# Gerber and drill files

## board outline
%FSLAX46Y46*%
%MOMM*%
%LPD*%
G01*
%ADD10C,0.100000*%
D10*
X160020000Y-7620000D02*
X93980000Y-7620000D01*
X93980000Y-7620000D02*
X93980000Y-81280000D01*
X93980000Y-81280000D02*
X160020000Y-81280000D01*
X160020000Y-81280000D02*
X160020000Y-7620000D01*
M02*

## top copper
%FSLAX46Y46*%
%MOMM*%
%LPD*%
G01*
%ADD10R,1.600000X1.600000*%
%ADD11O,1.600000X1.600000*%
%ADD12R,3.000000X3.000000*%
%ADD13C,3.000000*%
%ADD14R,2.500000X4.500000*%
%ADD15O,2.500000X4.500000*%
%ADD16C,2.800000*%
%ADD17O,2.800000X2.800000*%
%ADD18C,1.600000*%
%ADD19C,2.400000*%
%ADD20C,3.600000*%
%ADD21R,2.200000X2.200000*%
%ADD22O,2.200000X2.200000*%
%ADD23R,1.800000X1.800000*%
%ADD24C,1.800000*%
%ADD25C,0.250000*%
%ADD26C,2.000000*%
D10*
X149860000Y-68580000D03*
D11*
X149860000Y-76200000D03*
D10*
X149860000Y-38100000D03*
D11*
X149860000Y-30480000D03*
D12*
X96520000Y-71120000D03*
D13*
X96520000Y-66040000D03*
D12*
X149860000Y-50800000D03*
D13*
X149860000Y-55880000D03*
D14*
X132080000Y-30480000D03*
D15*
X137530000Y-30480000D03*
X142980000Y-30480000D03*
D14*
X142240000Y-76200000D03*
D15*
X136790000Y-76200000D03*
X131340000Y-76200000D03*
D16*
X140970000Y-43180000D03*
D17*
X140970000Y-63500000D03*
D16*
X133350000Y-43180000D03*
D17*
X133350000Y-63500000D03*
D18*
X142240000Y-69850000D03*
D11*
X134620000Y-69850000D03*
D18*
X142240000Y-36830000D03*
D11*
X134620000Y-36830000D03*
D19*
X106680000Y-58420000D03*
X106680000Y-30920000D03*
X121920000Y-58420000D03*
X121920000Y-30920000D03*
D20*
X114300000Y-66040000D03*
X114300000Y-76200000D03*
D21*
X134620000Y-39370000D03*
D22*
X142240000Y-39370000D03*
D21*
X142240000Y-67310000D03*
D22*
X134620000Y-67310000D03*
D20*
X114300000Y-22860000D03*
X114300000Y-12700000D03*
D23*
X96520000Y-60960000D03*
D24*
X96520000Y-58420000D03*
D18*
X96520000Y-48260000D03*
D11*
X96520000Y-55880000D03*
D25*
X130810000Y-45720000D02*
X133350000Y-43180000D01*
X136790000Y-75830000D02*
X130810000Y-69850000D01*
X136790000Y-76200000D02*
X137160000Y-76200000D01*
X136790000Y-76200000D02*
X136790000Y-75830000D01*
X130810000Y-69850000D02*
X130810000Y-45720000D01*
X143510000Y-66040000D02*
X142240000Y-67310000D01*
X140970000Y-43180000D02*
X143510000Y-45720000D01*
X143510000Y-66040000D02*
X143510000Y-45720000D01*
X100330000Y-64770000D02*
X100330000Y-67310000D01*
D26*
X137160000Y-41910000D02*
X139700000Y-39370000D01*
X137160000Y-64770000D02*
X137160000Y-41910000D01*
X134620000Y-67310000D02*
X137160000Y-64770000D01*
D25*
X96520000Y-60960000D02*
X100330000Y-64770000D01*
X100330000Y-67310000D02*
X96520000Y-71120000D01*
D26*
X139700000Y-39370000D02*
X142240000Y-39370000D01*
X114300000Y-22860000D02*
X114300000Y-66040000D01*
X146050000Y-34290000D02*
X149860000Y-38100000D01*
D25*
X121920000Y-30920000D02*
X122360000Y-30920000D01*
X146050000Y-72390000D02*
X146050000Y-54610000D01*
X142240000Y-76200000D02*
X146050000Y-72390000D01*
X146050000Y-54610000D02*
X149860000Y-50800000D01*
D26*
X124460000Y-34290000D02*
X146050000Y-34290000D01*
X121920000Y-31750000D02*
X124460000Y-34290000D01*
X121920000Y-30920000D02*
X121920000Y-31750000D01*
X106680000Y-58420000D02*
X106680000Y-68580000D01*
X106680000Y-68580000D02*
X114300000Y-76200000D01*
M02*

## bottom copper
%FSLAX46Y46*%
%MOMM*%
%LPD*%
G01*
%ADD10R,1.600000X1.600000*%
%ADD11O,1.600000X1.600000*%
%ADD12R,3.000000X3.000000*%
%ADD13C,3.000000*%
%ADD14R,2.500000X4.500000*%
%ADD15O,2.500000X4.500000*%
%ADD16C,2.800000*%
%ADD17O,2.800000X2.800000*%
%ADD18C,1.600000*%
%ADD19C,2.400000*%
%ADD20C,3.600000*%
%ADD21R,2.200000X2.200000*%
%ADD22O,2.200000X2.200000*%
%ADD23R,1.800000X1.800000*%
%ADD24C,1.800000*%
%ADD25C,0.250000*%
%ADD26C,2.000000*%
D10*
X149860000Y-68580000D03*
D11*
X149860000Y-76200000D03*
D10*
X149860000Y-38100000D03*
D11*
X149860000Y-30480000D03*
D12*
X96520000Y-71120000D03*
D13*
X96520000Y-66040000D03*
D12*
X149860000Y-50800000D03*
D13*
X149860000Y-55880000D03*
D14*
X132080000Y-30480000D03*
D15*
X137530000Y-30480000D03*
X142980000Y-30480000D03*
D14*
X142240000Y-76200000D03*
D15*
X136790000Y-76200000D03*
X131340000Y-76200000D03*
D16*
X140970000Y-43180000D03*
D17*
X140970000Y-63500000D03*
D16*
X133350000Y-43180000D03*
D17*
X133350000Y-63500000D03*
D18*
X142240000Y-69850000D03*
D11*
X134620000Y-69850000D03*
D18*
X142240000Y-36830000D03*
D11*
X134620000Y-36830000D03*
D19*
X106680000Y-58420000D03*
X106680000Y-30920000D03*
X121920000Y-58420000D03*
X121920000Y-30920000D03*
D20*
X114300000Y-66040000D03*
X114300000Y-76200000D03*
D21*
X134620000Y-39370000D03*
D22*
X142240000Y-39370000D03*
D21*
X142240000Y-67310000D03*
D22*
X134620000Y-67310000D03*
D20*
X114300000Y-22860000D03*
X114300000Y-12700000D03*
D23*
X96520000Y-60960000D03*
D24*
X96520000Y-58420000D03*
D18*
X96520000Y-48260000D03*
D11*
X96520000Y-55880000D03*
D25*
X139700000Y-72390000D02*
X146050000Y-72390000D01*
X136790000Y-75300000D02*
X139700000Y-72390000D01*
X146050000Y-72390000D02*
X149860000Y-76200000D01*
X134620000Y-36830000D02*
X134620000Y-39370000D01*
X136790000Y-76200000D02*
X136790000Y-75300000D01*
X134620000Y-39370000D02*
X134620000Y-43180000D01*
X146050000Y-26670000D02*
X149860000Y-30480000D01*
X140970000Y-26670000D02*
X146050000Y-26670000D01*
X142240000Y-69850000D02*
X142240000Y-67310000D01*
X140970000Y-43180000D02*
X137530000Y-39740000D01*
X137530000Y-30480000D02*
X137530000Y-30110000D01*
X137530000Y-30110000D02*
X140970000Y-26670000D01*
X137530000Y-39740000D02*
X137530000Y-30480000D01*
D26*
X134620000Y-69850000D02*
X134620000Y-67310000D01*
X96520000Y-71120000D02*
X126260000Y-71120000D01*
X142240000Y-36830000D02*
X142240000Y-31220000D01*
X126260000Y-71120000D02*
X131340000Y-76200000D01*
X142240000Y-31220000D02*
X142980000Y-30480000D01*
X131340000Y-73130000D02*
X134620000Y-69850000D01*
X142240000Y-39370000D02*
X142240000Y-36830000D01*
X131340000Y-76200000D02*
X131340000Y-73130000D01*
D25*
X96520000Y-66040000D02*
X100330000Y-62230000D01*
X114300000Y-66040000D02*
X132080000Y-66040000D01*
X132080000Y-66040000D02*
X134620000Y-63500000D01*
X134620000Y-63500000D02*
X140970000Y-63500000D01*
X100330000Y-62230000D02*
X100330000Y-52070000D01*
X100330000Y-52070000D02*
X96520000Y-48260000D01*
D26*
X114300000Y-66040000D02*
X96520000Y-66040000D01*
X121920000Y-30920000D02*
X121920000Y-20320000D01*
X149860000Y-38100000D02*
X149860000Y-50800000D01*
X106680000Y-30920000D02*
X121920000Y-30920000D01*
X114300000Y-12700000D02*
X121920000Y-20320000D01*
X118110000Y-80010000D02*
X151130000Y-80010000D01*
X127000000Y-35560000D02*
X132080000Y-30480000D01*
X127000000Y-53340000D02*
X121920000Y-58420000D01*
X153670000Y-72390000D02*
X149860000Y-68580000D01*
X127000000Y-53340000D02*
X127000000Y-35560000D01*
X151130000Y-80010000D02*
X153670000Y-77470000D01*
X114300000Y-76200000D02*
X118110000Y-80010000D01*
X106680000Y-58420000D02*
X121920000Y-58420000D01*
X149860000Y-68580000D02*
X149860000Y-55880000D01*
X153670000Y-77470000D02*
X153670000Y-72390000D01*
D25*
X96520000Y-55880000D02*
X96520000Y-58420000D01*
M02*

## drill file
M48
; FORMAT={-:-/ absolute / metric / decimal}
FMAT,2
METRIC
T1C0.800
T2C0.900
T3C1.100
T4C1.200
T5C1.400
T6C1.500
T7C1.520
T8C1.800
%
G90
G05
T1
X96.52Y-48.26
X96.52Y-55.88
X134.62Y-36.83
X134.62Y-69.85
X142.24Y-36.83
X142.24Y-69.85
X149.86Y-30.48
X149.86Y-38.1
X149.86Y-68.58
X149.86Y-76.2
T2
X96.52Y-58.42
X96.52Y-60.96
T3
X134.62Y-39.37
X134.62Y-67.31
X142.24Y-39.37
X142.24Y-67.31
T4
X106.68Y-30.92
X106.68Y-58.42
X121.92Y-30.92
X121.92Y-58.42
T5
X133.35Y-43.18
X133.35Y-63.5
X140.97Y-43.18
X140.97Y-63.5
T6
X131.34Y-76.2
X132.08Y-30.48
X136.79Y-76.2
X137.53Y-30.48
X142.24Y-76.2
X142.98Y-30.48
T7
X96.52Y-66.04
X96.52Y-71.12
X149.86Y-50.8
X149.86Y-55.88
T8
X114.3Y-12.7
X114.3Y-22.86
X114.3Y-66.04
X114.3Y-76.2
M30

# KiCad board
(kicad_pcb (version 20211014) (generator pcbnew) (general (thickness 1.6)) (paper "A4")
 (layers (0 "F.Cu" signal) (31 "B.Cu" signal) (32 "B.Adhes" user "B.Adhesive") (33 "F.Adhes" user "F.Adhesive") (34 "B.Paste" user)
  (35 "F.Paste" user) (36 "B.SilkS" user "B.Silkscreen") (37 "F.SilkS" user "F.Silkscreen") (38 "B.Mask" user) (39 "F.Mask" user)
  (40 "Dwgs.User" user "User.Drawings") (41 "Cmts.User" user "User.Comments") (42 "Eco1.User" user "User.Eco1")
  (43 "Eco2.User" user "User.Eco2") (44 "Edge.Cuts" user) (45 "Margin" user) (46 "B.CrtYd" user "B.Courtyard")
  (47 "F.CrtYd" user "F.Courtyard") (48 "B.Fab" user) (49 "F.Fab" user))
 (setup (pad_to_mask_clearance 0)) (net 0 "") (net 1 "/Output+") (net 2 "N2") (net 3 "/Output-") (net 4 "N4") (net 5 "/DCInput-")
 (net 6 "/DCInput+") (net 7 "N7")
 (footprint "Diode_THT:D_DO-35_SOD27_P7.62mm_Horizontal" (layer "F.Cu") (at 149.86 68.58 -90)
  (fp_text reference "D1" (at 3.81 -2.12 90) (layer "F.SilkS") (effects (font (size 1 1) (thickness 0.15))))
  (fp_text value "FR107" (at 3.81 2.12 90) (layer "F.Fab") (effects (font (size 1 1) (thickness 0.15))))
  (pad "1" thru_hole rect (at 0 0 270) (size 1.6 1.6) (drill 0.8) (layers *.Cu *.Mask) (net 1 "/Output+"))
  (pad "2" thru_hole oval (at 7.62 0 270) (size 1.6 1.6) (drill 0.8) (layers *.Cu *.Mask) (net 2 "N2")))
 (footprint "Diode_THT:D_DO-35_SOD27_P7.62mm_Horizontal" (layer "F.Cu") (at 149.86 38.1 90)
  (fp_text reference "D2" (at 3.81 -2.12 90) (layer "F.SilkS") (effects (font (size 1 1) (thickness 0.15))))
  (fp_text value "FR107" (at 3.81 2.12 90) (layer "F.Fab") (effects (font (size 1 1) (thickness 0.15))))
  (pad "1" thru_hole rect (at 0 0 90) (size 1.6 1.6) (drill 0.8) (layers *.Cu *.Mask) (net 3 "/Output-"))
  (pad "2" thru_hole oval (at 7.62 0 90) (size 1.6 1.6) (drill 0.8) (layers *.Cu *.Mask) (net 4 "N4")))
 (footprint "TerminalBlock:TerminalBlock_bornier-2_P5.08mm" (layer "F.Cu") (at 96.52 71.12 90)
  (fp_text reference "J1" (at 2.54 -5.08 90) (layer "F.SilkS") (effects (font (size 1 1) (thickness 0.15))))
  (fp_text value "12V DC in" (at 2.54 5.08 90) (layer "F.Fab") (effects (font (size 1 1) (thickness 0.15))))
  (pad "1" thru_hole rect (at 0 0 90) (size 3 3) (drill 1.52) (layers *.Cu *.Mask) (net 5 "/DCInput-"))
  (pad "2" thru_hole circle (at 5.08 0 90) (size 3 3) (drill 1.52) (layers *.Cu *.Mask) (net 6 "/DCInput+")))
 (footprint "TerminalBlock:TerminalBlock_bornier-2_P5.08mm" (layer "F.Cu") (at 149.86 50.8 -90)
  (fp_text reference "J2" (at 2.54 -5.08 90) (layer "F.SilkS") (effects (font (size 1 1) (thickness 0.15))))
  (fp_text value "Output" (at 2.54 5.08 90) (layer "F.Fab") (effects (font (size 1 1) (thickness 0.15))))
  (pad "1" thru_hole rect (at 0 0 270) (size 3 3) (drill 1.52) (layers *.Cu *.Mask) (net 3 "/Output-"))
  (pad "2" thru_hole circle (at 5.08 0 270) (size 3 3) (drill 1.52) (layers *.Cu *.Mask) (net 1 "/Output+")))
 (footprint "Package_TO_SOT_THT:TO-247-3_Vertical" (layer "F.Cu") (at 132.08 30.48)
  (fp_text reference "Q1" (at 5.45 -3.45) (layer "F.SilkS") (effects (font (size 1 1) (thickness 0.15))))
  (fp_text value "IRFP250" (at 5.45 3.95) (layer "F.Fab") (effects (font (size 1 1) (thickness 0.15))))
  (pad "1" thru_hole rect (at 0 0) (size 2.5 4.5) (drill 1.5) (layers *.Cu *.Mask) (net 1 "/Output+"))
  (pad "2" thru_hole oval (at 5.45 0) (size 2.5 4.5) (drill 1.5) (layers *.Cu *.Mask) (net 4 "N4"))
  (pad "3" thru_hole oval (at 10.9 0) (size 2.5 4.5) (drill 1.5) (layers *.Cu *.Mask) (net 5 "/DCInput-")))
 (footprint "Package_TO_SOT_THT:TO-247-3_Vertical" (layer "F.Cu") (at 142.24 76.2 180)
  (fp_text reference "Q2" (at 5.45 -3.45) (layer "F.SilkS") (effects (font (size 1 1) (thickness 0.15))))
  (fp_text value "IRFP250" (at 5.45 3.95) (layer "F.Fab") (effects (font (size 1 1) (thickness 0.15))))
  (pad "1" thru_hole rect (at 0 0 180) (size 2.5 4.5) (drill 1.5) (layers *.Cu *.Mask) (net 3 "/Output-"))
  (pad "2" thru_hole oval (at 5.45 0 180) (size 2.5 4.5) (drill 1.5) (layers *.Cu *.Mask) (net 2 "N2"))
  (pad "3" thru_hole oval (at 10.9 0 180) (size 2.5 4.5) (drill 1.5) (layers *.Cu *.Mask) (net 5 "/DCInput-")))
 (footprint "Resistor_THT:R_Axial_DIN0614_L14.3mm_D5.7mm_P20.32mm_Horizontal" (layer "F.Cu") (at 140.97 43.18 -90)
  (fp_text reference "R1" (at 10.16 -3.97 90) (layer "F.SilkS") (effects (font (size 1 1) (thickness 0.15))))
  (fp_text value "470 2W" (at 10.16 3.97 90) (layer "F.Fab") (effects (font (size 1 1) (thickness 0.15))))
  (pad "1" thru_hole circle (at 0 0 270) (size 2.8 2.8) (drill 1.4) (layers *.Cu *.Mask) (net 4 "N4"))
  (pad "2" thru_hole oval (at 20.32 0 270) (size 2.8 2.8) (drill 1.4) (layers *.Cu *.Mask) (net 6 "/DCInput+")))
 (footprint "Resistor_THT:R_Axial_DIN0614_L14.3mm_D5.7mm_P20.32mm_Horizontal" (layer "F.Cu") (at 133.35 43.18 -90)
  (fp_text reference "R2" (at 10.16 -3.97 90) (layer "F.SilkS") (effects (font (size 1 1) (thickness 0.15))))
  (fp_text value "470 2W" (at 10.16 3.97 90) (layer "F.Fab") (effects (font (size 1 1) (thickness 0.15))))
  (pad "1" thru_hole circle (at 0 0 270) (size 2.8 2.8) (drill 1.4) (layers *.Cu *.Mask) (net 2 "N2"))
  (pad "2" thru_hole oval (at 20.32 0 270) (size 2.8 2.8) (drill 1.4) (layers *.Cu *.Mask) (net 6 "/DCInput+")))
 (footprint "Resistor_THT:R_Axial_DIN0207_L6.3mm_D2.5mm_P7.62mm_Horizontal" (layer "F.Cu") (at 142.24 69.85 180)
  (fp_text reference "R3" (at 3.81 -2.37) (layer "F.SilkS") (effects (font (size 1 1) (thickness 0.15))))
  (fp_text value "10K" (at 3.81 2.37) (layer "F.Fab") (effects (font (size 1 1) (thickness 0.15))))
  (pad "1" thru_hole circle (at 0 0 180) (size 1.6 1.6) (drill 0.8) (layers *.Cu *.Mask) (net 4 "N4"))
  (pad "2" thru_hole oval (at 7.62 0 180) (size 1.6 1.6) (drill 0.8) (layers *.Cu *.Mask) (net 5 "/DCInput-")))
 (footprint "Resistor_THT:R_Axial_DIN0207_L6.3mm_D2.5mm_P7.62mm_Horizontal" (layer "F.Cu") (at 142.24 36.83 180)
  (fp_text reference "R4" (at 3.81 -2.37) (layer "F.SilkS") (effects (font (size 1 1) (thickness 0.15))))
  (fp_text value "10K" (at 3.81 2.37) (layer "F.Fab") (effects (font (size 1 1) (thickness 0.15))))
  (pad "1" thru_hole circle (at 0 0 180) (size 1.6 1.6) (drill 0.8) (layers *.Cu *.Mask) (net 5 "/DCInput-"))
  (pad "2" thru_hole oval (at 7.62 0 180) (size 1.6 1.6) (drill 0.8) (layers *.Cu *.Mask) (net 2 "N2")))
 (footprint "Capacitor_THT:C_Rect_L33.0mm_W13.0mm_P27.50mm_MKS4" (layer "F.Cu") (at 106.68 58.42 90)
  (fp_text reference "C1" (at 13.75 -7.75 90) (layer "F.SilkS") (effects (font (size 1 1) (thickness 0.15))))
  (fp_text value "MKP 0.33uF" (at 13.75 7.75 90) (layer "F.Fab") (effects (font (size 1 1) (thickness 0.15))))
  (pad "1" thru_hole circle (at 0 0 90) (size 2.4 2.4) (drill 1.2) (layers *.Cu *.Mask) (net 1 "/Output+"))
  (pad "2" thru_hole circle (at 27.5 0 90) (size 2.4 2.4) (drill 1.2) (layers *.Cu *.Mask) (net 3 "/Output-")))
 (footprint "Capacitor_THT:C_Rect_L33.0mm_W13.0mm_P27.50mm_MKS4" (layer "F.Cu") (at 121.92 58.42 90)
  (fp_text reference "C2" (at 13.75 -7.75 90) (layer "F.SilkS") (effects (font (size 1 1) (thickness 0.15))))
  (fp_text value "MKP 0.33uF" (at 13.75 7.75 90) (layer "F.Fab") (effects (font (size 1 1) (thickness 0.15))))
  (pad "1" thru_hole circle (at 0 0 90) (size 2.4 2.4) (drill 1.2) (layers *.Cu *.Mask) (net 1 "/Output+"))
  (pad "2" thru_hole circle (at 27.5 0 90) (size 2.4 2.4) (drill 1.2) (layers *.Cu *.Mask) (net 3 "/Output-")))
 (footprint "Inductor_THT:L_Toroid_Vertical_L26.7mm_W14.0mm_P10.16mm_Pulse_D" (layer "F.Cu") (at 114.3 66.04)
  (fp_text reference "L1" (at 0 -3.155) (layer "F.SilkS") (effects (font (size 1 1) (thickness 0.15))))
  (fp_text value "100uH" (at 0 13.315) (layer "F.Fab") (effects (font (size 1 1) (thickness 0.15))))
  (pad "1" thru_hole circle (at 0 0) (size 3.6 3.6) (drill 1.8) (layers *.Cu *.Mask) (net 6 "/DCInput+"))
  (pad "2" thru_hole circle (at 0 10.16) (size 3.6 3.6) (drill 1.8) (layers *.Cu *.Mask) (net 1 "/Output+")))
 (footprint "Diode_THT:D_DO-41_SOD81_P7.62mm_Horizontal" (layer "F.Cu") (at 134.62 39.37)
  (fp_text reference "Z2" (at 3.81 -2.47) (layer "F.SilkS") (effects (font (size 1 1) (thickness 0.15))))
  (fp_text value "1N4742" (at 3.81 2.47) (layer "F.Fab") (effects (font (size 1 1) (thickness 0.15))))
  (pad "1" thru_hole rect (at 0 0) (size 2.2 2.2) (drill 1.1) (layers *.Cu *.Mask) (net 2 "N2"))
  (pad "2" thru_hole oval (at 7.62 0) (size 2.2 2.2) (drill 1.1) (layers *.Cu *.Mask) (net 5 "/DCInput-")))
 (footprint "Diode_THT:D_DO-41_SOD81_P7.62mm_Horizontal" (layer "F.Cu") (at 142.24 67.31 180)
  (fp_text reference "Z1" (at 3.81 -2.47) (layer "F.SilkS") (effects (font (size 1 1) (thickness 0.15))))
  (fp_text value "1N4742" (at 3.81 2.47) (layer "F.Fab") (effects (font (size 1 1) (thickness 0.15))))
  (pad "1" thru_hole rect (at 0 0 180) (size 2.2 2.2) (drill 1.1) (layers *.Cu *.Mask) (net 4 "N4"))
  (pad "2" thru_hole oval (at 7.62 0 180) (size 2.2 2.2) (drill 1.1) (layers *.Cu *.Mask) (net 5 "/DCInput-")))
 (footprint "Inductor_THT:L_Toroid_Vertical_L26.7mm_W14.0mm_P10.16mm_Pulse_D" (layer "F.Cu") (at 114.3 22.86 180)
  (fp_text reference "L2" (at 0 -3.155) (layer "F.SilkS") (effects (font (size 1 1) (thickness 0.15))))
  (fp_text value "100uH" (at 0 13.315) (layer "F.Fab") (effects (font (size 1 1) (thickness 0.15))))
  (pad "1" thru_hole circle (at 0 0 180) (size 3.6 3.6) (drill 1.8) (layers *.Cu *.Mask) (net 6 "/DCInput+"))
  (pad "2" thru_hole circle (at 0 10.16 180) (size 3.6 3.6) (drill 1.8) (layers *.Cu *.Mask) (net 3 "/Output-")))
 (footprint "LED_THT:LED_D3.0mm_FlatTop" (layer "F.Cu") (at 96.52 60.96 90)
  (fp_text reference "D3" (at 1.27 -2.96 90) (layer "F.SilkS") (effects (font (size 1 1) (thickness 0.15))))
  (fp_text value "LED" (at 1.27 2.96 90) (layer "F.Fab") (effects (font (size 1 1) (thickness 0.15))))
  (pad "1" thru_hole rect (at 0 0 90) (size 1.8 1.8) (drill 0.9) (layers *.Cu *.Mask) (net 5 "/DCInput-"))
  (pad "2" thru_hole circle (at 2.54 0 90) (size 1.8 1.8) (drill 0.9) (layers *.Cu *.Mask) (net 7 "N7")))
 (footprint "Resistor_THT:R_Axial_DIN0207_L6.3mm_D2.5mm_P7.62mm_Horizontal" (layer "F.Cu") (at 96.52 48.26 -90)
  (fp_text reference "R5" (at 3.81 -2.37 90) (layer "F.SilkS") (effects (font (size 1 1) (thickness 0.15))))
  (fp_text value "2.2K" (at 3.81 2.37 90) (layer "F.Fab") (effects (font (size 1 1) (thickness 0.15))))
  (pad "1" thru_hole circle (at 0 0 270) (size 1.6 1.6) (drill 0.8) (layers *.Cu *.Mask) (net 6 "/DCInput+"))
  (pad "2" thru_hole oval (at 7.62 0 270) (size 1.6 1.6) (drill 0.8) (layers *.Cu *.Mask) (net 7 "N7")))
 (gr_line (start 160.02 7.62) (end 93.98 7.62) (layer "Edge.Cuts") (width 0.1))
 (gr_line (start 93.98 7.62) (end 93.98 81.28) (layer "Edge.Cuts") (width 0.1))
 (gr_line (start 93.98 81.28) (end 160.02 81.28) (layer "Edge.Cuts") (width 0.1))
 (gr_line (start 160.02 81.28) (end 160.02 7.62) (layer "Edge.Cuts") (width 0.1))
 (segment (start 130.81 45.72) (end 133.35 43.18) (width 0.25) (layer "F.Cu") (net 2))
 (segment (start 136.79 75.83) (end 130.81 69.85) (width 0.25) (layer "F.Cu") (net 2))
 (segment (start 136.79 76.2) (end 137.16 76.2) (width 0.25) (layer "F.Cu") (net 2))
 (segment (start 136.79 76.2) (end 136.79 75.83) (width 0.25) (layer "F.Cu") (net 2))
 (segment (start 130.81 69.85) (end 130.81 45.72) (width 0.25) (layer "F.Cu") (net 2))
 (segment (start 139.7 72.39) (end 146.05 72.39) (width 0.25) (layer "B.Cu") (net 2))
 (segment (start 136.79 75.3) (end 139.7 72.39) (width 0.25) (layer "B.Cu") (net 2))
 (segment (start 146.05 72.39) (end 149.86 76.2) (width 0.25) (layer "B.Cu") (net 2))
 (segment (start 134.62 36.83) (end 134.62 39.37) (width 0.25) (layer "B.Cu") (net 2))
 (segment (start 136.79 76.2) (end 136.79 75.3) (width 0.25) (layer "B.Cu") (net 2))
 (segment (start 134.62 39.37) (end 134.62 43.18) (width 0.25) (layer "B.Cu") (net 2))
 (segment (start 143.51 66.04) (end 142.24 67.31) (width 0.25) (layer "F.Cu") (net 4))
 (segment (start 140.97 43.18) (end 143.51 45.72) (width 0.25) (layer "F.Cu") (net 4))
 (segment (start 143.51 66.04) (end 143.51 45.72) (width 0.25) (layer "F.Cu") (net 4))
 (segment (start 146.05 26.67) (end 149.86 30.48) (width 0.25) (layer "B.Cu") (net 4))
 (segment (start 140.97 26.67) (end 146.05 26.67) (width 0.25) (layer "B.Cu") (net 4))
 (segment (start 142.24 69.85) (end 142.24 67.31) (width 0.25) (layer "B.Cu") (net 4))
 (segment (start 140.97 43.18) (end 137.53 39.74) (width 0.25) (layer "B.Cu") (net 4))
 (segment (start 137.53 30.48) (end 137.53 30.11) (width 0.25) (layer "B.Cu") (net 4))
 (segment (start 137.53 30.11) (end 140.97 26.67) (width 0.25) (layer "B.Cu") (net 4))
 (segment (start 137.53 39.74) (end 137.53 30.48) (width 0.25) (layer "B.Cu") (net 4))
 (segment (start 100.33 64.77) (end 100.33 67.31) (width 0.25) (layer "F.Cu") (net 5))
 (segment (start 137.16 41.91) (end 139.7 39.37) (width 2) (layer "F.Cu") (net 5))
 (segment (start 137.16 64.77) (end 137.16 41.91) (width 2) (layer "F.Cu") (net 5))
 (segment (start 134.62 67.31) (end 137.16 64.77) (width 2) (layer "F.Cu") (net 5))
 (segment (start 96.52 60.96) (end 100.33 64.77) (width 0.25) (layer "F.Cu") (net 5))
 (segment (start 100.33 67.31) (end 96.52 71.12) (width 0.25) (layer "F.Cu") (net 5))
 (segment (start 139.7 39.37) (end 142.24 39.37) (width 2) (layer "F.Cu") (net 5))
 (segment (start 134.62 69.85) (end 134.62 67.31) (width 2) (layer "B.Cu") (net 5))
 (segment (start 96.52 71.12) (end 126.26 71.12) (width 2) (layer "B.Cu") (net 5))
 (segment (start 142.24 36.83) (end 142.24 31.22) (width 2) (layer "B.Cu") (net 5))
 (segment (start 126.26 71.12) (end 131.34 76.2) (width 2) (layer "B.Cu") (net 5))
 (segment (start 142.24 31.22) (end 142.98 30.48) (width 2) (layer "B.Cu") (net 5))
 (segment (start 131.34 73.13) (end 134.62 69.85) (width 2) (layer "B.Cu") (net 5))
 (segment (start 142.24 39.37) (end 142.24 36.83) (width 2) (layer "B.Cu") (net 5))
 (segment (start 131.34 76.2) (end 131.34 73.13) (width 2) (layer "B.Cu") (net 5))
 (segment (start 114.3 22.86) (end 114.3 66.04) (width 2) (layer "F.Cu") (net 6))
 (segment (start 96.52 66.04) (end 100.33 62.23) (width 0.25) (layer "B.Cu") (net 6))
 (segment (start 114.3 66.04) (end 132.08 66.04) (width 0.25) (layer "B.Cu") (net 6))
 (segment (start 132.08 66.04) (end 134.62 63.5) (width 0.25) (layer "B.Cu") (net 6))
 (segment (start 134.62 63.5) (end 140.97 63.5) (width 0.25) (layer "B.Cu") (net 6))
 (segment (start 100.33 62.23) (end 100.33 52.07) (width 0.25) (layer "B.Cu") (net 6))
 (segment (start 100.33 52.07) (end 96.52 48.26) (width 0.25) (layer "B.Cu") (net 6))
 (segment (start 114.3 66.04) (end 96.52 66.04) (width 2) (layer "B.Cu") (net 6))
 (segment (start 146.05 34.29) (end 149.86 38.1) (width 2) (layer "F.Cu") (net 3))
 (segment (start 121.92 30.92) (end 122.36 30.92) (width 0.25) (layer "F.Cu") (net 3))
 (segment (start 146.05 72.39) (end 146.05 54.61) (width 0.25) (layer "F.Cu") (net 3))
 (segment (start 142.24 76.2) (end 146.05 72.39) (width 0.25) (layer "F.Cu") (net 3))
 (segment (start 146.05 54.61) (end 149.86 50.8) (width 0.25) (layer "F.Cu") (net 3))
 (segment (start 124.46 34.29) (end 146.05 34.29) (width 2) (layer "F.Cu") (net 3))
 (segment (start 121.92 31.75) (end 124.46 34.29) (width 2) (layer "F.Cu") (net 3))
 (segment (start 121.92 30.92) (end 121.92 31.75) (width 2) (layer "F.Cu") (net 3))
 (segment (start 121.92 30.92) (end 121.92 20.32) (width 2) (layer "B.Cu") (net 3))
 (segment (start 149.86 38.1) (end 149.86 50.8) (width 2) (layer "B.Cu") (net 3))
 (segment (start 106.68 30.92) (end 121.92 30.92) (width 2) (layer "B.Cu") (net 3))
 (segment (start 114.3 12.7) (end 121.92 20.32) (width 2) (layer "B.Cu") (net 3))
 (segment (start 106.68 58.42) (end 106.68 68.58) (width 2) (layer "F.Cu") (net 1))
 (segment (start 106.68 68.58) (end 114.3 76.2) (width 2) (layer "F.Cu") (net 1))
 (segment (start 118.11 80.01) (end 151.13 80.01) (width 2) (layer "B.Cu") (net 1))
 (segment (start 127 35.56) (end 132.08 30.48) (width 2) (layer "B.Cu") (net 1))
 (segment (start 127 53.34) (end 121.92 58.42) (width 2) (layer "B.Cu") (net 1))
 (segment (start 153.67 72.39) (end 149.86 68.58) (width 2) (layer "B.Cu") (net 1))
 (segment (start 127 53.34) (end 127 35.56) (width 2) (layer "B.Cu") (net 1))
 (segment (start 151.13 80.01) (end 153.67 77.47) (width 2) (layer "B.Cu") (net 1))
 (segment (start 114.3 76.2) (end 118.11 80.01) (width 2) (layer "B.Cu") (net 1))
 (segment (start 106.68 58.42) (end 121.92 58.42) (width 2) (layer "B.Cu") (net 1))
 (segment (start 149.86 68.58) (end 149.86 55.88) (width 2) (layer "B.Cu") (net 1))
 (segment (start 153.67 77.47) (end 153.67 72.39) (width 2) (layer "B.Cu") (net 1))
 (segment (start 96.52 55.88) (end 96.52 58.42) (width 0.25) (layer "B.Cu") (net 7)))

